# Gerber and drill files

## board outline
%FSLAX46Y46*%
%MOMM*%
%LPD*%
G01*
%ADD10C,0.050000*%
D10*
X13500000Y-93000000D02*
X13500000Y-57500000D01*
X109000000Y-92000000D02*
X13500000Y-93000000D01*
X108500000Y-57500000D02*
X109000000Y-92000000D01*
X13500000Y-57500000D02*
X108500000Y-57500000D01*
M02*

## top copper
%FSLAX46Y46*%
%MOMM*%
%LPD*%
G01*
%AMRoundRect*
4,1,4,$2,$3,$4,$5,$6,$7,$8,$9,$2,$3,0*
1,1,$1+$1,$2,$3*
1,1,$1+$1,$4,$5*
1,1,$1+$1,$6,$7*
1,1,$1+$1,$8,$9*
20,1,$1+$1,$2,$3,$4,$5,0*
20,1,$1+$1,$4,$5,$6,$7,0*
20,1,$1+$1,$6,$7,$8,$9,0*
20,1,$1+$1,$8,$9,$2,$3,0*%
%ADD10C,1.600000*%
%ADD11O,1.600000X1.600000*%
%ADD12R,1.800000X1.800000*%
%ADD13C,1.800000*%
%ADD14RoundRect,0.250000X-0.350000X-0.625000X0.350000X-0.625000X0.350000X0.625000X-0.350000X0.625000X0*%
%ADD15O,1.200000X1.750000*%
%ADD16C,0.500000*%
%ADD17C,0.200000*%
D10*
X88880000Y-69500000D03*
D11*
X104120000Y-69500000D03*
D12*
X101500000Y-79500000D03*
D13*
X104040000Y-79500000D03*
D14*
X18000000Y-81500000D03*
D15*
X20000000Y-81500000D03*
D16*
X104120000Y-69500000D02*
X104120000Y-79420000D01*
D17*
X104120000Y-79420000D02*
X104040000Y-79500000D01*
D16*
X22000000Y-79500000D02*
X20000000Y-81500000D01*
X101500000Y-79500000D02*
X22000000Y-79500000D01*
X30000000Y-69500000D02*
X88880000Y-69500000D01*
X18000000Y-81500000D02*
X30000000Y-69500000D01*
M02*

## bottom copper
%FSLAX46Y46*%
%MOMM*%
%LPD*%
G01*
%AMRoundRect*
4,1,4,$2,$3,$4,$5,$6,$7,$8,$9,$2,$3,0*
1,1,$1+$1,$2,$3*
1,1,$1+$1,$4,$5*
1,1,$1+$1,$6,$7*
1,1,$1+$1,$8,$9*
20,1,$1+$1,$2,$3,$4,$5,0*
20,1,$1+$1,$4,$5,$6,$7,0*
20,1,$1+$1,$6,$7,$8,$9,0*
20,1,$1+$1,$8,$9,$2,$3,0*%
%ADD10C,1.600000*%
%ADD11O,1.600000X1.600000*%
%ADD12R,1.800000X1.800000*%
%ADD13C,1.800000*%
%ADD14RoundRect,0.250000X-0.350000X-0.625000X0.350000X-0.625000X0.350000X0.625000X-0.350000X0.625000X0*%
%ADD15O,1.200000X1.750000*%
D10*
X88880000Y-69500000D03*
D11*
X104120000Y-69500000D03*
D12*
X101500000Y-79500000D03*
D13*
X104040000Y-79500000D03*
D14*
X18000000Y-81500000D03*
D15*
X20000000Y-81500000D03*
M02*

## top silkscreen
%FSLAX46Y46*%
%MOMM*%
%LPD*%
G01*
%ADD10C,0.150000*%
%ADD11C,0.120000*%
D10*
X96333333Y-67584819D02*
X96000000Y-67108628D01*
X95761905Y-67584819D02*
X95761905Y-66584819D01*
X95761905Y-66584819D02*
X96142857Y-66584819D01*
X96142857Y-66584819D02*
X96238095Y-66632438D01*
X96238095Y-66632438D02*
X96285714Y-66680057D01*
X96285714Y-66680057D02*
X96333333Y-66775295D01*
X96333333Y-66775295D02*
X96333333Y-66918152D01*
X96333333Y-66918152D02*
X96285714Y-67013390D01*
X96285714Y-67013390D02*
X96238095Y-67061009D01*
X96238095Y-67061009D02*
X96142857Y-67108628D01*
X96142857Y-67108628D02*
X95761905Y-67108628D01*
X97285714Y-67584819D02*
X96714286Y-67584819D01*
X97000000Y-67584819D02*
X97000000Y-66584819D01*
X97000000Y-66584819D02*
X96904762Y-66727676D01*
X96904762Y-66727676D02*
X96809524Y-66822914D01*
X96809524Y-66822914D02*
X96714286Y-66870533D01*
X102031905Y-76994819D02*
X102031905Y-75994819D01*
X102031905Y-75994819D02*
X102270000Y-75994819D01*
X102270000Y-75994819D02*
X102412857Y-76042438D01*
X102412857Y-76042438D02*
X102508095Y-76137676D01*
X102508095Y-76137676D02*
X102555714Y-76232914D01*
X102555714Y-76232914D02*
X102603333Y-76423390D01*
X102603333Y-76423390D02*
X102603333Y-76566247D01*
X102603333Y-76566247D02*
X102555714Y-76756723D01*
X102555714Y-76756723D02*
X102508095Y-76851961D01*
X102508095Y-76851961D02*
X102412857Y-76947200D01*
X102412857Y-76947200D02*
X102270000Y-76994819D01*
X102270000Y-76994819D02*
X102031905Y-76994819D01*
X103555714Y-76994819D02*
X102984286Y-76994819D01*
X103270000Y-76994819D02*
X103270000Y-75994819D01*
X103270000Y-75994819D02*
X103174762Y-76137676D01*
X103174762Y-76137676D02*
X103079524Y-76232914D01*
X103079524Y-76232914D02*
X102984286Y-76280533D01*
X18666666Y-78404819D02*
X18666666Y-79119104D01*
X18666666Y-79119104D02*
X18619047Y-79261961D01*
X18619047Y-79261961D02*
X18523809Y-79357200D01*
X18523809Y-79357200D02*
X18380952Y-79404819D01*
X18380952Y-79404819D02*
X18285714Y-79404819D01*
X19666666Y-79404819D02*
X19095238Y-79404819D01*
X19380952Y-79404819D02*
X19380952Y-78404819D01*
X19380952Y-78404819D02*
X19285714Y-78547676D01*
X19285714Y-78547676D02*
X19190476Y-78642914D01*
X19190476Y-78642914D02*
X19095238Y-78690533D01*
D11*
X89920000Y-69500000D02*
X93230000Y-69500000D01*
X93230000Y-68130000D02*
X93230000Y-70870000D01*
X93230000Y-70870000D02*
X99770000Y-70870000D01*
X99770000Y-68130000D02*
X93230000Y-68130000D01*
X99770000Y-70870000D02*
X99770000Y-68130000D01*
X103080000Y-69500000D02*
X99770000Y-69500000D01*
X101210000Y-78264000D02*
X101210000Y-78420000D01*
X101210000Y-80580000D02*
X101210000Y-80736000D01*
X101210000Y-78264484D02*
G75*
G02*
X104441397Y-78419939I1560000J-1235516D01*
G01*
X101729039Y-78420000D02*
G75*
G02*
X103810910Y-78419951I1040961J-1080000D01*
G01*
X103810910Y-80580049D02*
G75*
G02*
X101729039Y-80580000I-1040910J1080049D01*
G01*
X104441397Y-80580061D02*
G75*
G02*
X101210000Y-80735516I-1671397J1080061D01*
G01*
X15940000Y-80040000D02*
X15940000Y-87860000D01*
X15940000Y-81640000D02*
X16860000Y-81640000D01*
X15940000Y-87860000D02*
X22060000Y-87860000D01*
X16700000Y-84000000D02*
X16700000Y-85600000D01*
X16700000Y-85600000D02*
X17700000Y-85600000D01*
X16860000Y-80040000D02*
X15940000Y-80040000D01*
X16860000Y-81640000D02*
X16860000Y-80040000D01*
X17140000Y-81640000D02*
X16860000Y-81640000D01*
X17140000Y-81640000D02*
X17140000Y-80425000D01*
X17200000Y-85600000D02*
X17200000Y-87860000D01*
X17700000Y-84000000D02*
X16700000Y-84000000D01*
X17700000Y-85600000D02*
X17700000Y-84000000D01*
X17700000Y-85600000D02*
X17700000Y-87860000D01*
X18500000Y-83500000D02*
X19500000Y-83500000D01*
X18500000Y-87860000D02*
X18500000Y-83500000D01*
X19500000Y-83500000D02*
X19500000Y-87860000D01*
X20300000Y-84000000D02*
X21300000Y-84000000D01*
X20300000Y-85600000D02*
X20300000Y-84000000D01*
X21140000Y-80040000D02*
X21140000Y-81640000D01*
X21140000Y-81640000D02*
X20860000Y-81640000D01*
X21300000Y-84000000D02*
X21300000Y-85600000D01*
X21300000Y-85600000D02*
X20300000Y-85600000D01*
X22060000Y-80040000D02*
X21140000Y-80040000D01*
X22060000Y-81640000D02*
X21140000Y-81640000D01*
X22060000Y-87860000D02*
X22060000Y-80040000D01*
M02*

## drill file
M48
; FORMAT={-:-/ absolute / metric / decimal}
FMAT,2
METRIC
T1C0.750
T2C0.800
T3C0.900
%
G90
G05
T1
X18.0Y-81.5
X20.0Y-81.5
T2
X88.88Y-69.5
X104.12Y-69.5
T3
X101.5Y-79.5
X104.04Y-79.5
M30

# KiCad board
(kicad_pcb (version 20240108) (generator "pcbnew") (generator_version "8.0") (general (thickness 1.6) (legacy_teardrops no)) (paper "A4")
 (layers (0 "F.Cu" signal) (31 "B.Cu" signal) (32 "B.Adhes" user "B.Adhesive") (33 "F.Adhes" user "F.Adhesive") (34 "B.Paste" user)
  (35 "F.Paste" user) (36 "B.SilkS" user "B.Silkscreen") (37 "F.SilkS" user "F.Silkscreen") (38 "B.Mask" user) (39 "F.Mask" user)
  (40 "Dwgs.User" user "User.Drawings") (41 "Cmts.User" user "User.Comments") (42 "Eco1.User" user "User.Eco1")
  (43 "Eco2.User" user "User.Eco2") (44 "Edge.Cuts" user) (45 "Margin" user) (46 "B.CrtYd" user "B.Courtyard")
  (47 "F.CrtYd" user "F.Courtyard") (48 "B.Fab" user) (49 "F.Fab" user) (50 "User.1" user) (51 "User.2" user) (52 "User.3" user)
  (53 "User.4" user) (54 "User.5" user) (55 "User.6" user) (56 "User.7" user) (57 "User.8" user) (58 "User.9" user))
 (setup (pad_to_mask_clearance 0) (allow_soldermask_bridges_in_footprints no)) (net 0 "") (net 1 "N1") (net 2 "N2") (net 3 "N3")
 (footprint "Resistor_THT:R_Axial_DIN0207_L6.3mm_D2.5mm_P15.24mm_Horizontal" (layer "F.Cu") (at 88.88 69.5)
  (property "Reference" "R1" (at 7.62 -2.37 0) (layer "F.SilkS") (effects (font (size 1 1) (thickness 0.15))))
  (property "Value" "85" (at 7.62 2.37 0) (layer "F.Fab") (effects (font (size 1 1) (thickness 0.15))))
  (fp_line (start 1.04 0) (end 4.35 0) (stroke (width 0.12) (type solid)) (layer "F.SilkS"))
  (fp_line (start 4.35 -1.37) (end 4.35 1.37) (stroke (width 0.12) (type solid)) (layer "F.SilkS"))
  (fp_line (start 4.35 1.37) (end 10.89 1.37) (stroke (width 0.12) (type solid)) (layer "F.SilkS"))
  (fp_line (start 10.89 -1.37) (end 4.35 -1.37) (stroke (width 0.12) (type solid)) (layer "F.SilkS"))
  (fp_line (start 10.89 1.37) (end 10.89 -1.37) (stroke (width 0.12) (type solid)) (layer "F.SilkS"))
  (fp_line (start 14.2 0) (end 10.89 0) (stroke (width 0.12) (type solid)) (layer "F.SilkS"))
  (pad "1" thru_hole circle (at 0 0) (size 1.6 1.6) (drill 0.8) (layers "*.Cu" "*.Mask") (remove_unused_layers no) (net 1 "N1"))
  (pad "2" thru_hole oval (at 15.24 0) (size 1.6 1.6) (drill 0.8) (layers "*.Cu" "*.Mask") (remove_unused_layers no) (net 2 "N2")))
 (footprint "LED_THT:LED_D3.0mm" (layer "F.Cu") (at 101.5 79.5)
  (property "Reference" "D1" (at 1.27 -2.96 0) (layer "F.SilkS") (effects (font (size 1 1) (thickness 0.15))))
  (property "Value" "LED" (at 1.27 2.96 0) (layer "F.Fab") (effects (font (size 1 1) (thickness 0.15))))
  (fp_line (start -0.29 -1.236) (end -0.29 -1.08) (stroke (width 0.12) (type solid)) (layer "F.SilkS"))
  (fp_line (start -0.29 1.08) (end -0.29 1.236) (stroke (width 0.12) (type solid)) (layer "F.SilkS"))
  (fp_arc (start -0.29 -1.235516) (mid 1.365624 -1.987701) (end 2.941397 -1.080061) (stroke (width 0.12) (type solid)) (layer "F.SilkS"))
  (fp_arc (start 0.229039 -1.08) (mid 1.269965 -1.5) (end 2.31091 -1.080049) (stroke (width 0.12) (type solid)) (layer "F.SilkS"))
  (fp_arc (start 2.31091 1.080049) (mid 1.269965 1.5) (end 0.229039 1.08) (stroke (width 0.12) (type solid)) (layer "F.SilkS"))
  (fp_arc (start 2.941397 1.080061) (mid 1.365624 1.987701) (end -0.29 1.235516) (stroke (width 0.12) (type solid)) (layer "F.SilkS"))
  (pad "1" thru_hole rect (at 0 0) (size 1.8 1.8) (drill 0.9) (layers "*.Cu" "*.Mask") (remove_unused_layers no) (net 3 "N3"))
  (pad "2" thru_hole circle (at 2.54 0) (size 1.8 1.8) (drill 0.9) (layers "*.Cu" "*.Mask") (remove_unused_layers no) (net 2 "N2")))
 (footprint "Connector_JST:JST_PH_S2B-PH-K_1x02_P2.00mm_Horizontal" (layer "F.Cu") (at 18 81.5)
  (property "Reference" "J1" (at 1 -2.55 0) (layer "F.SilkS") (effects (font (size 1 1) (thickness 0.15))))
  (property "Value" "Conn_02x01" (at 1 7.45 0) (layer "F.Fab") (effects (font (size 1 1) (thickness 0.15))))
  (fp_line (start -2.06 -1.46) (end -2.06 6.36) (stroke (width 0.12) (type solid)) (layer "F.SilkS"))
  (fp_line (start -2.06 0.14) (end -1.14 0.14) (stroke (width 0.12) (type solid)) (layer "F.SilkS"))
  (fp_line (start -2.06 6.36) (end 4.06 6.36) (stroke (width 0.12) (type solid)) (layer "F.SilkS"))
  (fp_line (start -1.3 2.5) (end -1.3 4.1) (stroke (width 0.12) (type solid)) (layer "F.SilkS"))
  (fp_line (start -1.3 4.1) (end -0.3 4.1) (stroke (width 0.12) (type solid)) (layer "F.SilkS"))
  (fp_line (start -1.14 -1.46) (end -2.06 -1.46) (stroke (width 0.12) (type solid)) (layer "F.SilkS"))
  (fp_line (start -1.14 0.14) (end -1.14 -1.46) (stroke (width 0.12) (type solid)) (layer "F.SilkS"))
  (fp_line (start -0.86 0.14) (end -1.14 0.14) (stroke (width 0.12) (type solid)) (layer "F.SilkS"))
  (fp_line (start -0.86 0.14) (end -0.86 -1.075) (stroke (width 0.12) (type solid)) (layer "F.SilkS"))
  (fp_line (start -0.8 4.1) (end -0.8 6.36) (stroke (width 0.12) (type solid)) (layer "F.SilkS"))
  (fp_line (start -0.3 2.5) (end -1.3 2.5) (stroke (width 0.12) (type solid)) (layer "F.SilkS"))
  (fp_line (start -0.3 4.1) (end -0.3 2.5) (stroke (width 0.12) (type solid)) (layer "F.SilkS"))
  (fp_line (start -0.3 4.1) (end -0.3 6.36) (stroke (width 0.12) (type solid)) (layer "F.SilkS"))
  (fp_line (start 0.5 2) (end 1.5 2) (stroke (width 0.12) (type solid)) (layer "F.SilkS"))
  (fp_line (start 0.5 6.36) (end 0.5 2) (stroke (width 0.12) (type solid)) (layer "F.SilkS"))
  (fp_line (start 1.5 2) (end 1.5 6.36) (stroke (width 0.12) (type solid)) (layer "F.SilkS"))
  (fp_line (start 2.3 2.5) (end 3.3 2.5) (stroke (width 0.12) (type solid)) (layer "F.SilkS"))
  (fp_line (start 2.3 4.1) (end 2.3 2.5) (stroke (width 0.12) (type solid)) (layer "F.SilkS"))
  (fp_line (start 3.14 -1.46) (end 3.14 0.14) (stroke (width 0.12) (type solid)) (layer "F.SilkS"))
  (fp_line (start 3.14 0.14) (end 2.86 0.14) (stroke (width 0.12) (type solid)) (layer "F.SilkS"))
  (fp_line (start 3.3 2.5) (end 3.3 4.1) (stroke (width 0.12) (type solid)) (layer "F.SilkS"))
  (fp_line (start 3.3 4.1) (end 2.3 4.1) (stroke (width 0.12) (type solid)) (layer "F.SilkS"))
  (fp_line (start 4.06 -1.46) (end 3.14 -1.46) (stroke (width 0.12) (type solid)) (layer "F.SilkS"))
  (fp_line (start 4.06 0.14) (end 3.14 0.14) (stroke (width 0.12) (type solid)) (layer "F.SilkS"))
  (fp_line (start 4.06 6.36) (end 4.06 -1.46) (stroke (width 0.12) (type solid)) (layer "F.SilkS"))
  (pad "1" thru_hole roundrect (at 0 0) (size 1.2 1.75) (drill 0.75) (layers "*.Cu" "*.Mask") (remove_unused_layers no)
   (roundrect_rratio 0.208333) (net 1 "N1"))
  (pad "2" thru_hole oval (at 2 0) (size 1.2 1.75) (drill 0.75) (layers "*.Cu" "*.Mask") (remove_unused_layers no) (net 3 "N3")))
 (gr_line (start 13.5 93) (end 13.5 57.5) (stroke (width 0.05) (type default)) (layer "Edge.Cuts"))
 (gr_line (start 109 92) (end 13.5 93) (stroke (width 0.05) (type default)) (layer "Edge.Cuts"))
 (gr_line (start 108.5 57.5) (end 109 92) (stroke (width 0.05) (type default)) (layer "Edge.Cuts"))
 (gr_line (start 13.5 57.5) (end 108.5 57.5) (stroke (width 0.05) (type default)) (layer "Edge.Cuts"))
 (segment (start 104.12 69.5) (end 104.12 79.42) (width 0.5) (layer "F.Cu") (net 2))
 (segment (start 104.12 79.42) (end 104.04 79.5) (width 0.2) (layer "F.Cu") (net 2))
 (segment (start 22 79.5) (end 20 81.5) (width 0.5) (layer "F.Cu") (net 3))
 (segment (start 101.5 79.5) (end 22 79.5) (width 0.5) (layer "F.Cu") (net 3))
 (segment (start 30 69.5) (end 88.88 69.5) (width 0.5) (layer "F.Cu") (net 1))
 (segment (start 18 81.5) (end 30 69.5) (width 0.5) (layer "F.Cu") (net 1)))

